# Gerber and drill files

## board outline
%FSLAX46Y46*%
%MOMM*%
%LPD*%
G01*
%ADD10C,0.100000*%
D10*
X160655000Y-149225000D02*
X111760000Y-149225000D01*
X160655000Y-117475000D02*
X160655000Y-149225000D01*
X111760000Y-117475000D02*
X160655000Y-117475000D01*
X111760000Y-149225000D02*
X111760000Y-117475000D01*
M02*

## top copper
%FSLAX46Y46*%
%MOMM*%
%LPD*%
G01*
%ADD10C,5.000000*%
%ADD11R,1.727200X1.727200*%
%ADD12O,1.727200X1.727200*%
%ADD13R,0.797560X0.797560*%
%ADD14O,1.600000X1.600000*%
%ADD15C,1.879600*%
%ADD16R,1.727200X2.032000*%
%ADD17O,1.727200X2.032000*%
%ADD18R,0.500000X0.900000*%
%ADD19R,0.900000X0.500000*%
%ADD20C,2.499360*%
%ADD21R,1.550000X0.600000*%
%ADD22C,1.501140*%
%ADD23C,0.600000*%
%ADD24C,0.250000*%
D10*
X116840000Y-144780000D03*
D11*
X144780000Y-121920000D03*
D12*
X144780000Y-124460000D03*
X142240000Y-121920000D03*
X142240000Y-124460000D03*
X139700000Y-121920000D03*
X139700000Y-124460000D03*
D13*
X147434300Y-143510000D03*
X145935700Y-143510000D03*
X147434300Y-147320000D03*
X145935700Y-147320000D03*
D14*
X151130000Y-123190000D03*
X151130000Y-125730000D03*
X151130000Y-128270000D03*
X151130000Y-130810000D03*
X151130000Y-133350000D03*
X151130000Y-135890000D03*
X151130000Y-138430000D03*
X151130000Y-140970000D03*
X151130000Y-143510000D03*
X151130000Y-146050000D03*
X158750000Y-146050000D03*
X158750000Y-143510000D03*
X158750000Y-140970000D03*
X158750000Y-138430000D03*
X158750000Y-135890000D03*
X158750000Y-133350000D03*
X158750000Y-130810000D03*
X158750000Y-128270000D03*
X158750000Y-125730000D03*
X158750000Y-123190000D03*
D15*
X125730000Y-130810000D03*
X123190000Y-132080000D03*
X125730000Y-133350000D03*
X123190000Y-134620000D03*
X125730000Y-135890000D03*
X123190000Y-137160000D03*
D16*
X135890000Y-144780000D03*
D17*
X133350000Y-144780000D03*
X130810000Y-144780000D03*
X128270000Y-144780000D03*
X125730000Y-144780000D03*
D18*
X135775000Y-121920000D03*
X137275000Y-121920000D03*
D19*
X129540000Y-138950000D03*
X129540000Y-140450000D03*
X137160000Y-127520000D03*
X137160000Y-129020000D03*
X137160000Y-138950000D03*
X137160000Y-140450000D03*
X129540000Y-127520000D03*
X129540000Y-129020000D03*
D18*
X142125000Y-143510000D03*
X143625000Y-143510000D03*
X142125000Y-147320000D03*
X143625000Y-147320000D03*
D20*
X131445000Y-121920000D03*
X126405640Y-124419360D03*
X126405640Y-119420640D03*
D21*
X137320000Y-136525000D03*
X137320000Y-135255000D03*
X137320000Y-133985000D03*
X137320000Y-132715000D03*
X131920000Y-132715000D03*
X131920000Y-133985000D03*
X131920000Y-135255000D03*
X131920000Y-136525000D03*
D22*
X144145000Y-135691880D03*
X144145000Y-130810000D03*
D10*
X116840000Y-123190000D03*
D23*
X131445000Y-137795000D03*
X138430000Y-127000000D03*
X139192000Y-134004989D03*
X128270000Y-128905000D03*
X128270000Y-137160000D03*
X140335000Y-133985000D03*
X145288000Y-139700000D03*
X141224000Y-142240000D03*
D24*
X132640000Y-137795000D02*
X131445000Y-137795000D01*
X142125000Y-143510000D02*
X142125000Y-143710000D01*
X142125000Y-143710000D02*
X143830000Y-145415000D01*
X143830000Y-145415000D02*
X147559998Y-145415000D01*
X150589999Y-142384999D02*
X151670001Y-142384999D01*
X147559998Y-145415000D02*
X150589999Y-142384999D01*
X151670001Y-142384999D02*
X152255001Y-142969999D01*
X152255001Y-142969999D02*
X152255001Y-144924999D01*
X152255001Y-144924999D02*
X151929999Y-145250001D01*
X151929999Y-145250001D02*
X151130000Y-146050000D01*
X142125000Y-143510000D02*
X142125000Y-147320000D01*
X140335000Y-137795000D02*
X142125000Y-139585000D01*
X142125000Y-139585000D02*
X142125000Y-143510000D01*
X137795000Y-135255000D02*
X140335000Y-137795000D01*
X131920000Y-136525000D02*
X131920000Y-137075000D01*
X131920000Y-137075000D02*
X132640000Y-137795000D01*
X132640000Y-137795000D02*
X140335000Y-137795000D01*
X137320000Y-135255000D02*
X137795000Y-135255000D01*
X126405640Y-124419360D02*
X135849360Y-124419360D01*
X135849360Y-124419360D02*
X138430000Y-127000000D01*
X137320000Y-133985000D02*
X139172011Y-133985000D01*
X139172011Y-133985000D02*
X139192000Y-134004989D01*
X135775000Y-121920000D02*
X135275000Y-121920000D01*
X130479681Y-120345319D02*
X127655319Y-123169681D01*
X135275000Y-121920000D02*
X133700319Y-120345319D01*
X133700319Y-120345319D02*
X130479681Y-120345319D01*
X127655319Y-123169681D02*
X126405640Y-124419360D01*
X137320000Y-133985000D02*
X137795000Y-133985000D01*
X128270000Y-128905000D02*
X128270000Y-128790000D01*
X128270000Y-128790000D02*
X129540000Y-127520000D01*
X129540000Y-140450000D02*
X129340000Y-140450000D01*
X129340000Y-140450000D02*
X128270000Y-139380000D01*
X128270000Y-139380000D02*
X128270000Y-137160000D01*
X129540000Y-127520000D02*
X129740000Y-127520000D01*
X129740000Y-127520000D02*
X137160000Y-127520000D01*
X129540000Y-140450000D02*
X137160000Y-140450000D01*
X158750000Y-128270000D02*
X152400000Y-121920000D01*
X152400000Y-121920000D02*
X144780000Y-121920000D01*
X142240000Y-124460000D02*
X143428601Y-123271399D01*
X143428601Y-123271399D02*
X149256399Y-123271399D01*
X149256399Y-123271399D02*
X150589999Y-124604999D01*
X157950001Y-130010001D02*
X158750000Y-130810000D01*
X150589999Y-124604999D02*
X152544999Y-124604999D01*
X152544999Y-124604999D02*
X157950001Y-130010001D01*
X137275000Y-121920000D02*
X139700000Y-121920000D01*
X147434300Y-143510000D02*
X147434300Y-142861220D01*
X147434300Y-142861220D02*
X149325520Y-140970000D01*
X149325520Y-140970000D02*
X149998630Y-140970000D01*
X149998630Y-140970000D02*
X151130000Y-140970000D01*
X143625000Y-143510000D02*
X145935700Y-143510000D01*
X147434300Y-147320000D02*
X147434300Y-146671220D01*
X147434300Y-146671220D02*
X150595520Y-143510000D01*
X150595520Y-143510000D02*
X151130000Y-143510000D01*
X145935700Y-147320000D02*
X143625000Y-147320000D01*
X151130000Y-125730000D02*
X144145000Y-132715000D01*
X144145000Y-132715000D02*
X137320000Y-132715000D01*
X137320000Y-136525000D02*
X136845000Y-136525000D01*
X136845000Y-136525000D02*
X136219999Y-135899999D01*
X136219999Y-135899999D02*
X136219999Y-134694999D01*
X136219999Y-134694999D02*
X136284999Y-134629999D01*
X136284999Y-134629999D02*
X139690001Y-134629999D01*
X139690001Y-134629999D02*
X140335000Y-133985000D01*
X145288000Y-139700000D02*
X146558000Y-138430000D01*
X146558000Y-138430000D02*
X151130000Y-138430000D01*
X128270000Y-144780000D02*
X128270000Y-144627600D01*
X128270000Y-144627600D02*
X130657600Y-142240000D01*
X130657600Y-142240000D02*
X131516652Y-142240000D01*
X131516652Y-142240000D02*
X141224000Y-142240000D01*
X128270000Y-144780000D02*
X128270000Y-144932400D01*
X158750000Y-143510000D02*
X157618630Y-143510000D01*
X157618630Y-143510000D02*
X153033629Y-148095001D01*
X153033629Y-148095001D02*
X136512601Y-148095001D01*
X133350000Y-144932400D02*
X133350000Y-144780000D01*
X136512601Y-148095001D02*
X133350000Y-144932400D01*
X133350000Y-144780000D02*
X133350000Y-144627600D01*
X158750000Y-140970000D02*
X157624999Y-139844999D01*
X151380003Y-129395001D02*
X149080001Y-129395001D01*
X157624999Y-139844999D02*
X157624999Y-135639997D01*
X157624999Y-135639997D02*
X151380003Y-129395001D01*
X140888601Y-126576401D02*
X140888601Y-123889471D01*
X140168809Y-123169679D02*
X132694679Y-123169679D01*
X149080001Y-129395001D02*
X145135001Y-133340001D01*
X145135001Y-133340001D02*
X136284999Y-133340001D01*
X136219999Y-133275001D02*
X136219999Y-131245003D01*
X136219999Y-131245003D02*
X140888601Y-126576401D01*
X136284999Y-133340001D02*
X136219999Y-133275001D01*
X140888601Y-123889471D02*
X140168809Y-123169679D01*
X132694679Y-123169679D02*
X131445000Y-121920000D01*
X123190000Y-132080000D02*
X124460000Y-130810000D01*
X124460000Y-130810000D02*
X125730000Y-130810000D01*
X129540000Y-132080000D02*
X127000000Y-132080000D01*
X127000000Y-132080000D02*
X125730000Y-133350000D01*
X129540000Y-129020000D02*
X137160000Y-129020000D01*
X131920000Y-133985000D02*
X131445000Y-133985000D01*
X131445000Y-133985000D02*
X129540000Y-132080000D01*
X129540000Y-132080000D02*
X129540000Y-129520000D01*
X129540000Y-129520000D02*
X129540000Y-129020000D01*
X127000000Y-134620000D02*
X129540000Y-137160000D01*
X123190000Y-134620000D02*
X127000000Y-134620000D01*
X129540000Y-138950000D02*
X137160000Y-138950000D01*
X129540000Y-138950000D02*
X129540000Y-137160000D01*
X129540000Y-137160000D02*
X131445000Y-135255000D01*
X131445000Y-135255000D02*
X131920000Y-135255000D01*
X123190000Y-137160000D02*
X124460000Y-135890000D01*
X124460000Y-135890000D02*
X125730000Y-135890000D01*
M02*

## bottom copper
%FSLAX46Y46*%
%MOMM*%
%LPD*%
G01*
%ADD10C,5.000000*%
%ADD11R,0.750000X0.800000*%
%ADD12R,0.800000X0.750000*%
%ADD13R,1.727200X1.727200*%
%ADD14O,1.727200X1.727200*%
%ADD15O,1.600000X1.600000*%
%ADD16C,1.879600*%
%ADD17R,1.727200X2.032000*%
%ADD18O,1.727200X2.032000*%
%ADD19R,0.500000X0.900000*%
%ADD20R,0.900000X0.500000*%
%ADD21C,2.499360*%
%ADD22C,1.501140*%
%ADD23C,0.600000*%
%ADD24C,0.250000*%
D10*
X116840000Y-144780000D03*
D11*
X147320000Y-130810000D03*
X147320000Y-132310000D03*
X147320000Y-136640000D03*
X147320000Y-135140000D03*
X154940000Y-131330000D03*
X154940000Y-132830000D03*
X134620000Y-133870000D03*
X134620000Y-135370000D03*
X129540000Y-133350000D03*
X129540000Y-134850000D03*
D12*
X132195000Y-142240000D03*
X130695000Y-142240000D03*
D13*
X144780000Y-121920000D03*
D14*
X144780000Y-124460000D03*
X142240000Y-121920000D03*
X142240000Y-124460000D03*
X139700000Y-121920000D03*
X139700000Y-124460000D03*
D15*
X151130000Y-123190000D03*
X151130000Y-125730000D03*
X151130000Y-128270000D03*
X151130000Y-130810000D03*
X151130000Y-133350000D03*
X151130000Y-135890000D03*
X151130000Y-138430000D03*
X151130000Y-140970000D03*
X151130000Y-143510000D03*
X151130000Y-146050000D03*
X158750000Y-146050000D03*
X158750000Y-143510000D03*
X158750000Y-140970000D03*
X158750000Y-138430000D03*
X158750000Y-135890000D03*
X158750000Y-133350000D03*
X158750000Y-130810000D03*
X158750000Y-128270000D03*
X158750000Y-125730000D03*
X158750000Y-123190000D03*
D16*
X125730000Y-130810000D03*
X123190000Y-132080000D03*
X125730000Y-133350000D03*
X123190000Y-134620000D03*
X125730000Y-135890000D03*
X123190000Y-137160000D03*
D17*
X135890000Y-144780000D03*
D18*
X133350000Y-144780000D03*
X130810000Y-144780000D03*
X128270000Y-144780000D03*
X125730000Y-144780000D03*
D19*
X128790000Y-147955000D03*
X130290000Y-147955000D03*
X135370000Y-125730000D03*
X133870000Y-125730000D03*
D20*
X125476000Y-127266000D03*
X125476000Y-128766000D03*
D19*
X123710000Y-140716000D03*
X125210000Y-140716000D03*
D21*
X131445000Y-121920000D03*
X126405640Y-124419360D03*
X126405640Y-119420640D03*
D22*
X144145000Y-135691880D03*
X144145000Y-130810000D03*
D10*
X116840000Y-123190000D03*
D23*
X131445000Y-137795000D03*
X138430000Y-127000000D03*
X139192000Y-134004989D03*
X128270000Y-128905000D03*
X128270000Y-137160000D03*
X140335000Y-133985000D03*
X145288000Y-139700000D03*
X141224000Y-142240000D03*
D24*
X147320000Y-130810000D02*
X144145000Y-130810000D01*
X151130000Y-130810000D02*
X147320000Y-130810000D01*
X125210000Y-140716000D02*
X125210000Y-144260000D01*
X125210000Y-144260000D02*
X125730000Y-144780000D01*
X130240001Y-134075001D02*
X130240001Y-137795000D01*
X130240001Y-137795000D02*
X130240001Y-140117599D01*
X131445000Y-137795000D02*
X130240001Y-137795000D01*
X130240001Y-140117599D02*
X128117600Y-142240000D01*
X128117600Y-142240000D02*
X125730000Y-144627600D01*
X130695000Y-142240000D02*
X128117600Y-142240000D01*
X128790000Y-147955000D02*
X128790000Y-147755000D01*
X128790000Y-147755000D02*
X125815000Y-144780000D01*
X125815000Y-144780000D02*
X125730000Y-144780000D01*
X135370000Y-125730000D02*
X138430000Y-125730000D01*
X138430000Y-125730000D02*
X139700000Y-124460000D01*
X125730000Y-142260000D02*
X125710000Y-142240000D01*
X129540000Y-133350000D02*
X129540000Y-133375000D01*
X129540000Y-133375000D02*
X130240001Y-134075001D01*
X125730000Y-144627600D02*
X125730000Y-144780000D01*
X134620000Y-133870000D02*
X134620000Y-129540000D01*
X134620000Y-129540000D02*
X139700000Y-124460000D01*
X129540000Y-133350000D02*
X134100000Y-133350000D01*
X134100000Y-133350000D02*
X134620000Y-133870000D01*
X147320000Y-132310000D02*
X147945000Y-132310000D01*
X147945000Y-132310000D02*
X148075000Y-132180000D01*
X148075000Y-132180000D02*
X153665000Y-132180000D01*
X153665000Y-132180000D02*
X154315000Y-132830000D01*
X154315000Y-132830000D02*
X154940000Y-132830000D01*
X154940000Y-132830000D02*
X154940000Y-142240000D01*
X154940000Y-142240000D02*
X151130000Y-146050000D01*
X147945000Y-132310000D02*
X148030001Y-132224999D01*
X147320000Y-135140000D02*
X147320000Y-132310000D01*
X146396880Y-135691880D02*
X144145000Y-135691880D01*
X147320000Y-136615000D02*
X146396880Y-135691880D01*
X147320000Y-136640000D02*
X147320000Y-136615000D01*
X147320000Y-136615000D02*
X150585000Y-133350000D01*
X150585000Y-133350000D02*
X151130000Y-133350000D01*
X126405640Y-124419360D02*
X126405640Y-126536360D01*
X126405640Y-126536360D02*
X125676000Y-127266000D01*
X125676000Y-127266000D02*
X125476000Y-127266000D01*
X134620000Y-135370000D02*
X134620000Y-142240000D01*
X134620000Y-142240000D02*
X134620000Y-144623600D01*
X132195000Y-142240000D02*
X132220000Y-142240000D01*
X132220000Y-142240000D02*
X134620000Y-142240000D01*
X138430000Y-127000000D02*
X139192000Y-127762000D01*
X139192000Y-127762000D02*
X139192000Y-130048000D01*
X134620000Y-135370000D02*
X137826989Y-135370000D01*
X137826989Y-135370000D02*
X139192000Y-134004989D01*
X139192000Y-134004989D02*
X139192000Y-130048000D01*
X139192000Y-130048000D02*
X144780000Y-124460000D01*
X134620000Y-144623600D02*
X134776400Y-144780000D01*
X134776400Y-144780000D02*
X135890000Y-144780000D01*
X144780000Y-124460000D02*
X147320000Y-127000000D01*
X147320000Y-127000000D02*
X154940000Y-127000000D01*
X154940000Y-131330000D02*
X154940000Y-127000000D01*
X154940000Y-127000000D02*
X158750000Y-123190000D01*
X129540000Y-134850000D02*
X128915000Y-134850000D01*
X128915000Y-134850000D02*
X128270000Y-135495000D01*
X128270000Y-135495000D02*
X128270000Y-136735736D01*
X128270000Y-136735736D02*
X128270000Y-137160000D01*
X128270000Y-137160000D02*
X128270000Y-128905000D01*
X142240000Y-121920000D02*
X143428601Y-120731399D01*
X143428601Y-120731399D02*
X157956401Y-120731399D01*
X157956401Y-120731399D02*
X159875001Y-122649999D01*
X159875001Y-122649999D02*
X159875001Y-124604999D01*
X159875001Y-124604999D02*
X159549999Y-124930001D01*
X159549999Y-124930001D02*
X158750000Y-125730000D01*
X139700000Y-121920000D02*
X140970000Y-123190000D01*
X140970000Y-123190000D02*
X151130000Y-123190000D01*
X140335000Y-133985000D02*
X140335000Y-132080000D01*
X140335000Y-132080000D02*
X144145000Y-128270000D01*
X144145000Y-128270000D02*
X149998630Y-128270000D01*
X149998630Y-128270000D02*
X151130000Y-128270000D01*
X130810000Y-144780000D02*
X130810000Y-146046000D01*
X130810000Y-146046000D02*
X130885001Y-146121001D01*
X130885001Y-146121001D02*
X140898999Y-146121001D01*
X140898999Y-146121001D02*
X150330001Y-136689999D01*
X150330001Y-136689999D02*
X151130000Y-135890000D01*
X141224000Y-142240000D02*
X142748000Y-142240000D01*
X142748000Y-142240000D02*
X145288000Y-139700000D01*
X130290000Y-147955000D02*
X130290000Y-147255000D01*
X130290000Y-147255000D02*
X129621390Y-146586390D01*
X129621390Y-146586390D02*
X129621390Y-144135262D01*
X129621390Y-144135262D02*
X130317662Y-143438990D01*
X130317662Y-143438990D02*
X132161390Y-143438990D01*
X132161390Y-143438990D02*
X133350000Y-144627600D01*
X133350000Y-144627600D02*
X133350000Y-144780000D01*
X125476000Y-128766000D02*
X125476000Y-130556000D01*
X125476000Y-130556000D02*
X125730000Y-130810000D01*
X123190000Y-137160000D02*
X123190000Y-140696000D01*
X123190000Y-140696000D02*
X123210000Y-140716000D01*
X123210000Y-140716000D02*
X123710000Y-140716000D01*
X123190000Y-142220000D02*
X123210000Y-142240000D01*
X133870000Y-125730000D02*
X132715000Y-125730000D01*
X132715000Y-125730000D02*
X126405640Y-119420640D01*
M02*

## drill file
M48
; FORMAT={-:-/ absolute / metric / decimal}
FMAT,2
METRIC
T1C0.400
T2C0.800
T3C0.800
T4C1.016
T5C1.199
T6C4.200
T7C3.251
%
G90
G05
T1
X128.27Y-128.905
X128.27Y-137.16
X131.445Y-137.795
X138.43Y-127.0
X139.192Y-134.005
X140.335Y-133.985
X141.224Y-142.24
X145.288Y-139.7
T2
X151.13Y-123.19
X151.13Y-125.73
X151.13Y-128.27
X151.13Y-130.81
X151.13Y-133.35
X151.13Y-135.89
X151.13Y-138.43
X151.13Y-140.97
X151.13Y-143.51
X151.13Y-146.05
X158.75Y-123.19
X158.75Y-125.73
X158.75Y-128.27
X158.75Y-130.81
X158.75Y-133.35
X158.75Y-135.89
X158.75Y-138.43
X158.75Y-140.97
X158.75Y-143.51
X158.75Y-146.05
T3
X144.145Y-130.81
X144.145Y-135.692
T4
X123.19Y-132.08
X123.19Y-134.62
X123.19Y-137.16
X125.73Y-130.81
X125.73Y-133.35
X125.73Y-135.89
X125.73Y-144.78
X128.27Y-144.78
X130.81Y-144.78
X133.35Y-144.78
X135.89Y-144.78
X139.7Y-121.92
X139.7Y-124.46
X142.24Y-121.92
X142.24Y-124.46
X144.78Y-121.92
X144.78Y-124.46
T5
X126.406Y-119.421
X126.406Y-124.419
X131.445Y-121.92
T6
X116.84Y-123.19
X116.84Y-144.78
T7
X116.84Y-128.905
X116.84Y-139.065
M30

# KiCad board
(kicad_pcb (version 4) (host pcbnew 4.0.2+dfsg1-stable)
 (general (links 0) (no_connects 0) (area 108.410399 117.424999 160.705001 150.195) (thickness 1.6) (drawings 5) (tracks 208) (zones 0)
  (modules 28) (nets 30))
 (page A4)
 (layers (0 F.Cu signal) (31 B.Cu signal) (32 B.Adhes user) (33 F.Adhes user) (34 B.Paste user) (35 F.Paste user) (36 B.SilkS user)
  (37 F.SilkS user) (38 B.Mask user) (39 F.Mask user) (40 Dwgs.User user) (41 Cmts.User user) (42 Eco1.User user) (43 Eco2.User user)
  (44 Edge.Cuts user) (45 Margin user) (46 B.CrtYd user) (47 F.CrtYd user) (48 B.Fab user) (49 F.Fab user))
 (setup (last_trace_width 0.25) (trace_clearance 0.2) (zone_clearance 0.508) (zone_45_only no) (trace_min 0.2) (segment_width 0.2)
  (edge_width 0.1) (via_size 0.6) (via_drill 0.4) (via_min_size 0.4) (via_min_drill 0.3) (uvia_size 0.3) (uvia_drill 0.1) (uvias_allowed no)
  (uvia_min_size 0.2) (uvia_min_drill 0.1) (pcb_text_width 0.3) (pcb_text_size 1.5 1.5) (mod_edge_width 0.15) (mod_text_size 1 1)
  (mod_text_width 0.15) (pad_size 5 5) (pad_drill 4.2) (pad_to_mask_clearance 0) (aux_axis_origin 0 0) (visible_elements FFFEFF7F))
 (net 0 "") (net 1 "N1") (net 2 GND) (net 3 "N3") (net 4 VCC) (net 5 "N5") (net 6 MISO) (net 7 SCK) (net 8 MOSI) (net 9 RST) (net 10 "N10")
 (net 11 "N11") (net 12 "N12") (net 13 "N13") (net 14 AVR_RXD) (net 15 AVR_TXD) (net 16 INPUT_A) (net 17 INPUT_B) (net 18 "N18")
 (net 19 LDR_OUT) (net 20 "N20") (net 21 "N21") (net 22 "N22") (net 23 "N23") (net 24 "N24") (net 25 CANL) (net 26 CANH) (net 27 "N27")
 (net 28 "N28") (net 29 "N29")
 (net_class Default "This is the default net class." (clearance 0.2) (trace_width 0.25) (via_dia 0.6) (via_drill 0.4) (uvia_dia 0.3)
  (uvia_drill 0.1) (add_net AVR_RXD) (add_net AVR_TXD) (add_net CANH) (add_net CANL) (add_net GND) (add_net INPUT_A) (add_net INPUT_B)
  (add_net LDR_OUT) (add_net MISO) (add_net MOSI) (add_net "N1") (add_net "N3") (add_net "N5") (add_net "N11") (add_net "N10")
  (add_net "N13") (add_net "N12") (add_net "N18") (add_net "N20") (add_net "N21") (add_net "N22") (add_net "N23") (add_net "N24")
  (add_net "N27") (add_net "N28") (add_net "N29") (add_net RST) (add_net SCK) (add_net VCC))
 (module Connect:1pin (layer F.Cu) (at 116.84 144.78)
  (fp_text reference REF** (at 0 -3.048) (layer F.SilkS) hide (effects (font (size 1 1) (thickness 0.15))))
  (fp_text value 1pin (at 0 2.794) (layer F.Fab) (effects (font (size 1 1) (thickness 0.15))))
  (pad 1 thru_hole circle (at 0 0) (size 5 5) (drill 4.2) (layers *.Cu *.Mask F.SilkS)))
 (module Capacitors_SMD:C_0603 (layer B.Cu) (at 147.32 131.56 270)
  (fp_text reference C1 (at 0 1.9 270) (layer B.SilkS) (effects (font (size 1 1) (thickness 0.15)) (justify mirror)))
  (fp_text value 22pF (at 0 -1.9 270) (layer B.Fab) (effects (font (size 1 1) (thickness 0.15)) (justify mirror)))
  (pad 1 smd rect (at -0.75 0 270) (size 0.8 0.75) (layers B.Cu B.Paste B.Mask) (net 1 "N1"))
  (pad 2 smd rect (at 0.75 0 270) (size 0.8 0.75) (layers B.Cu B.Paste B.Mask) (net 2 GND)))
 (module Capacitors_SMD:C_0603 (layer B.Cu) (at 147.32 135.89 90)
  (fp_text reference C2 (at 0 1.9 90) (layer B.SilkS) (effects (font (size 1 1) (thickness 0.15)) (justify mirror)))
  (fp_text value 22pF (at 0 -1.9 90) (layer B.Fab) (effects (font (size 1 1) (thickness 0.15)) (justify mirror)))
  (pad 1 smd rect (at -0.75 0 90) (size 0.8 0.75) (layers B.Cu B.Paste B.Mask) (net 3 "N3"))
  (pad 2 smd rect (at 0.75 0 90) (size 0.8 0.75) (layers B.Cu B.Paste B.Mask) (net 2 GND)))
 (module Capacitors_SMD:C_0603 (layer B.Cu) (at 154.94 132.08 270)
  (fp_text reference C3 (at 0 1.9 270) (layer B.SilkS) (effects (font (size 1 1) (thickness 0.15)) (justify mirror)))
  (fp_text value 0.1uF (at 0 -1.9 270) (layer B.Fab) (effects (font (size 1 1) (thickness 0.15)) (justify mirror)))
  (pad 1 smd rect (at -0.75 0 270) (size 0.8 0.75) (layers B.Cu B.Paste B.Mask) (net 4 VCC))
  (pad 2 smd rect (at 0.75 0 270) (size 0.8 0.75) (layers B.Cu B.Paste B.Mask) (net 2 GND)))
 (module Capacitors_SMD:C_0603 (layer B.Cu) (at 134.62 134.62 270)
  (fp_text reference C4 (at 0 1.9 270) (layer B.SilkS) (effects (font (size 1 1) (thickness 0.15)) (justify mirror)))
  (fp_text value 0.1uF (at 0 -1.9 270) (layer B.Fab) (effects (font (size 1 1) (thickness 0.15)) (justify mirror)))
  (pad 1 smd rect (at -0.75 0 270) (size 0.8 0.75) (layers B.Cu B.Paste B.Mask) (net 2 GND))
  (pad 2 smd rect (at 0.75 0 270) (size 0.8 0.75) (layers B.Cu B.Paste B.Mask) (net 4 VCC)))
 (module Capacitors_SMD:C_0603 (layer B.Cu) (at 129.54 134.1 270)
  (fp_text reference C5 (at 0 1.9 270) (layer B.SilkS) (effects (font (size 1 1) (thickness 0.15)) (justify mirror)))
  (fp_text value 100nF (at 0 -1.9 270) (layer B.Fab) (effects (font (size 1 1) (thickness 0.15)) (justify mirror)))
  (pad 1 smd rect (at -0.75 0 270) (size 0.8 0.75) (layers B.Cu B.Paste B.Mask) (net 2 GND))
  (pad 2 smd rect (at 0.75 0 270) (size 0.8 0.75) (layers B.Cu B.Paste B.Mask) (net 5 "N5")))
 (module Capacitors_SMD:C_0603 (layer B.Cu) (at 131.445 142.24 180)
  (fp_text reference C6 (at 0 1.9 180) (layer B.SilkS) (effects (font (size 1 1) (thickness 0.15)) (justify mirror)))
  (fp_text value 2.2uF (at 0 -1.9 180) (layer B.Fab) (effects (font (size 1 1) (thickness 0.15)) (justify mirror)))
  (pad 1 smd rect (at -0.75 0 180) (size 0.8 0.75) (layers B.Cu B.Paste B.Mask) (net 4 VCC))
  (pad 2 smd rect (at 0.75 0 180) (size 0.8 0.75) (layers B.Cu B.Paste B.Mask) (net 2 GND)))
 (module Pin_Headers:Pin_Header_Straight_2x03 (layer F.Cu) (at 144.78 121.92 270)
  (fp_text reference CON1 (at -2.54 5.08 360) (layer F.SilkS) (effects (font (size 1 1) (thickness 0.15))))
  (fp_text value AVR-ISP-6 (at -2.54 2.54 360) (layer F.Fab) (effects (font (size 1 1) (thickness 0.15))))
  (pad 1 thru_hole rect (at 0 0 270) (size 1.7272 1.7272) (drill 1.016) (layers *.Cu *.Mask F.SilkS) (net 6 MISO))
  (pad 2 thru_hole oval (at 2.54 0 270) (size 1.7272 1.7272) (drill 1.016) (layers *.Cu *.Mask F.SilkS) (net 4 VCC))
  (pad 3 thru_hole oval (at 0 2.54 270) (size 1.7272 1.7272) (drill 1.016) (layers *.Cu *.Mask F.SilkS) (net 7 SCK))
  (pad 4 thru_hole oval (at 2.54 2.54 270) (size 1.7272 1.7272) (drill 1.016) (layers *.Cu *.Mask F.SilkS) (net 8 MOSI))
  (pad 5 thru_hole oval (at 0 5.08 270) (size 1.7272 1.7272) (drill 1.016) (layers *.Cu *.Mask F.SilkS) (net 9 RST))
  (pad 6 thru_hole oval (at 2.54 5.08 270) (size 1.7272 1.7272) (drill 1.016) (layers *.Cu *.Mask F.SilkS) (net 2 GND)))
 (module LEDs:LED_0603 (layer F.Cu) (at 146.685 143.51)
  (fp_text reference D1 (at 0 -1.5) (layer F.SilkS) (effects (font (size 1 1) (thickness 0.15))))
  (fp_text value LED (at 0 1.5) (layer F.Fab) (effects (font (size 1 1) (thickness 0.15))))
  (pad 2 smd rect (at 0.7493 0 180) (size 0.79756 0.79756) (layers F.Cu F.Paste F.Mask) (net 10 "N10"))
  (pad 1 smd rect (at -0.7493 0 180) (size 0.79756 0.79756) (layers F.Cu F.Paste F.Mask) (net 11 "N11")))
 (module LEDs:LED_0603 (layer F.Cu) (at 146.685 147.32)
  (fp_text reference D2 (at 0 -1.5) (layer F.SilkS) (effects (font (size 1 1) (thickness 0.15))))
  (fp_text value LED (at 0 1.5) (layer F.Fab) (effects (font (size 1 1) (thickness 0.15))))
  (pad 2 smd rect (at 0.7493 0 180) (size 0.79756 0.79756) (layers F.Cu F.Paste F.Mask) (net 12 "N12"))
  (pad 1 smd rect (at -0.7493 0 180) (size 0.79756 0.79756) (layers F.Cu F.Paste F.Mask) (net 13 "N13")))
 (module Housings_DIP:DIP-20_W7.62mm (layer F.Cu) (at 151.13 123.19)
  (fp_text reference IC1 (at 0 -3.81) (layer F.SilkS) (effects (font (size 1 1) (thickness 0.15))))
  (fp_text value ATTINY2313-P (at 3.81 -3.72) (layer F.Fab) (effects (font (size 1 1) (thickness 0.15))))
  (pad 1 thru_hole oval (at 0 0) (size 1.6 1.6) (drill 0.8) (layers *.Cu *.Mask F.SilkS) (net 9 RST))
  (pad 2 thru_hole oval (at 0 2.54) (size 1.6 1.6) (drill 0.8) (layers *.Cu *.Mask F.SilkS) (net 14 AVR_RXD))
  (pad 3 thru_hole oval (at 0 5.08) (size 1.6 1.6) (drill 0.8) (layers *.Cu *.Mask F.SilkS) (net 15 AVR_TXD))
  (pad 4 thru_hole oval (at 0 7.62) (size 1.6 1.6) (drill 0.8) (layers *.Cu *.Mask F.SilkS) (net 1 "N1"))
  (pad 5 thru_hole oval (at 0 10.16) (size 1.6 1.6) (drill 0.8) (layers *.Cu *.Mask F.SilkS) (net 3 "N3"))
  (pad 6 thru_hole oval (at 0 12.7) (size 1.6 1.6) (drill 0.8) (layers *.Cu *.Mask F.SilkS) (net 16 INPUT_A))
  (pad 7 thru_hole oval (at 0 15.24) (size 1.6 1.6) (drill 0.8) (layers *.Cu *.Mask F.SilkS) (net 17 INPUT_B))
  (pad 8 thru_hole oval (at 0 17.78) (size 1.6 1.6) (drill 0.8) (layers *.Cu *.Mask F.SilkS) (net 10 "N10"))
  (pad 9 thru_hole oval (at 0 20.32) (size 1.6 1.6) (drill 0.8) (layers *.Cu *.Mask F.SilkS) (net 12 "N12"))
  (pad 10 thru_hole oval (at 0 22.86) (size 1.6 1.6) (drill 0.8) (layers *.Cu *.Mask F.SilkS) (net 2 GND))
  (pad 11 thru_hole oval (at 7.62 22.86) (size 1.6 1.6) (drill 0.8) (layers *.Cu *.Mask F.SilkS) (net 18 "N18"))
  (pad 12 thru_hole oval (at 7.62 20.32) (size 1.6 1.6) (drill 0.8) (layers *.Cu *.Mask F.SilkS) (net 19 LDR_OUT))
  (pad 13 thru_hole oval (at 7.62 17.78) (size 1.6 1.6) (drill 0.8) (layers *.Cu *.Mask F.SilkS) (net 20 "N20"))
  (pad 14 thru_hole oval (at 7.62 15.24) (size 1.6 1.6) (drill 0.8) (layers *.Cu *.Mask F.SilkS) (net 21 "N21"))
  (pad 15 thru_hole oval (at 7.62 12.7) (size 1.6 1.6) (drill 0.8) (layers *.Cu *.Mask F.SilkS) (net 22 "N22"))
  (pad 16 thru_hole oval (at 7.62 10.16) (size 1.6 1.6) (drill 0.8) (layers *.Cu *.Mask F.SilkS) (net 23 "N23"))
  (pad 17 thru_hole oval (at 7.62 7.62) (size 1.6 1.6) (drill 0.8) (layers *.Cu *.Mask F.SilkS) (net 8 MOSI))
  (pad 18 thru_hole oval (at 7.62 5.08) (size 1.6 1.6) (drill 0.8) (layers *.Cu *.Mask F.SilkS) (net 6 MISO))
  (pad 19 thru_hole oval (at 7.62 2.54) (size 1.6 1.6) (drill 0.8) (layers *.Cu *.Mask F.SilkS) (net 7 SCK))
  (pad 20 thru_hole oval (at 7.62 0) (size 1.6 1.6) (drill 0.8) (layers *.Cu *.Mask F.SilkS) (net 4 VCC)))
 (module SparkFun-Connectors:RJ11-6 (layer F.Cu) (at 116.84 133.985 270)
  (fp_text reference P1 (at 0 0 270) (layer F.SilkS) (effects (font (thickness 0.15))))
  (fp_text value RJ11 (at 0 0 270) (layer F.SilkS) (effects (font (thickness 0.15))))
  (pad 1 thru_hole circle (at -3.175 -8.89 270) (size 1.8796 1.8796) (drill 1.016) (layers *.Cu *.Mask) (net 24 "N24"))
  (pad 2 thru_hole circle (at -1.905 -6.35 270) (size 1.8796 1.8796) (drill 1.016) (layers *.Cu *.Mask) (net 24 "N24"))
  (pad 3 thru_hole circle (at -0.635 -8.89 270) (size 1.8796 1.8796) (drill 1.016) (layers *.Cu *.Mask) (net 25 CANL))
  (pad 4 thru_hole circle (at 0.635 -6.35 270) (size 1.8796 1.8796) (drill 1.016) (layers *.Cu *.Mask) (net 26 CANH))
  (pad 5 thru_hole circle (at 1.905 -8.89 270) (size 1.8796 1.8796) (drill 1.016) (layers *.Cu *.Mask) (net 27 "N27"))
  (pad 6 thru_hole circle (at 3.175 -6.35 270) (size 1.8796 1.8796) (drill 1.016) (layers *.Cu *.Mask) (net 27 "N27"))
  (pad "" np_thru_hole circle (at -5.08 0 270) (size 3.2512 3.2512) (drill 3.2512) (layers *.Cu))
  (pad "" np_thru_hole circle (at 5.08 0 270) (size 3.2512 3.2512) (drill 3.2512) (layers *.Cu)))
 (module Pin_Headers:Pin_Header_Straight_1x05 (layer F.Cu) (at 135.89 144.78 270)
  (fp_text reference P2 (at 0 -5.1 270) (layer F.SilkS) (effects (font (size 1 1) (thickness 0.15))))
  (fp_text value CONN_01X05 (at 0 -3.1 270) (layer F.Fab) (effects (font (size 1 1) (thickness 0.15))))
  (pad 1 thru_hole rect (at 0 0 270) (size 2.032 1.7272) (drill 1.016) (layers *.Cu *.Mask F.SilkS) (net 4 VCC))
  (pad 2 thru_hole oval (at 0 2.54 270) (size 2.032 1.7272) (drill 1.016) (layers *.Cu *.Mask F.SilkS) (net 19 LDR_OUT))
  (pad 3 thru_hole oval (at 0 5.08 270) (size 2.032 1.7272) (drill 1.016) (layers *.Cu *.Mask F.SilkS) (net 16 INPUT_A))
  (pad 4 thru_hole oval (at 0 7.62 270) (size 2.032 1.7272) (drill 1.016) (layers *.Cu *.Mask F.SilkS) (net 17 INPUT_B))
  (pad 5 thru_hole oval (at 0 10.16 270) (size 2.032 1.7272) (drill 1.016) (layers *.Cu *.Mask F.SilkS) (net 2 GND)))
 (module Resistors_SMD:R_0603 (layer F.Cu) (at 136.525 121.92)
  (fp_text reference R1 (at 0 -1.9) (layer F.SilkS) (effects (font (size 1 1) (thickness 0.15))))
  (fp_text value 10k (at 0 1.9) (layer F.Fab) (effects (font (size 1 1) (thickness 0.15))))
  (pad 1 smd rect (at -0.75 0) (size 0.5 0.9) (layers F.Cu F.Paste F.Mask) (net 4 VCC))
  (pad 2 smd rect (at 0.75 0) (size 0.5 0.9) (layers F.Cu F.Paste F.Mask) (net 9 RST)))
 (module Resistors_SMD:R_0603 (layer B.Cu) (at 129.54 147.955)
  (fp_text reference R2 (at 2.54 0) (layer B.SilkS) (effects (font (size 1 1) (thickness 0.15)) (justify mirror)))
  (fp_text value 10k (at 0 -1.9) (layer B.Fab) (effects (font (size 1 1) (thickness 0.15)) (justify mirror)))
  (pad 1 smd rect (at -0.75 0) (size 0.5 0.9) (layers B.Cu B.Paste B.Mask) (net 2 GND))
  (pad 2 smd rect (at 0.75 0) (size 0.5 0.9) (layers B.Cu B.Paste B.Mask) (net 19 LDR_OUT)))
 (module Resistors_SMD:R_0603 (layer F.Cu) (at 129.54 139.7 270)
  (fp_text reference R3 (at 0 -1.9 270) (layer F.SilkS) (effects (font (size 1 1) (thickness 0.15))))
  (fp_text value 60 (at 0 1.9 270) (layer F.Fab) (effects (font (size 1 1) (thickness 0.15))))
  (pad 1 smd rect (at -0.75 0 270) (size 0.5 0.9) (layers F.Cu F.Paste F.Mask) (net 26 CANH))
  (pad 2 smd rect (at 0.75 0 270) (size 0.5 0.9) (layers F.Cu F.Paste F.Mask) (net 5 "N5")))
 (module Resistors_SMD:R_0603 (layer F.Cu) (at 137.16 128.27 270)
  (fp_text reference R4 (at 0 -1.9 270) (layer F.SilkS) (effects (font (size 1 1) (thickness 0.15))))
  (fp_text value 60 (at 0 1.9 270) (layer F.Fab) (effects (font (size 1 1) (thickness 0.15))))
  (pad 1 smd rect (at -0.75 0 270) (size 0.5 0.9) (layers F.Cu F.Paste F.Mask) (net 5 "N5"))
  (pad 2 smd rect (at 0.75 0 270) (size 0.5 0.9) (layers F.Cu F.Paste F.Mask) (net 25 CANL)))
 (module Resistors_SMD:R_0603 (layer F.Cu) (at 137.16 139.7 270)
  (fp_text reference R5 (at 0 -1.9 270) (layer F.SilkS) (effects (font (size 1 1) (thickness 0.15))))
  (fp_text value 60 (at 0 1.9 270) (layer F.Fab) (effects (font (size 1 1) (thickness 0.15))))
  (pad 1 smd rect (at -0.75 0 270) (size 0.5 0.9) (layers F.Cu F.Paste F.Mask) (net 26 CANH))
  (pad 2 smd rect (at 0.75 0 270) (size 0.5 0.9) (layers F.Cu F.Paste F.Mask) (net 5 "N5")))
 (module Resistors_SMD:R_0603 (layer F.Cu) (at 129.54 128.27 270)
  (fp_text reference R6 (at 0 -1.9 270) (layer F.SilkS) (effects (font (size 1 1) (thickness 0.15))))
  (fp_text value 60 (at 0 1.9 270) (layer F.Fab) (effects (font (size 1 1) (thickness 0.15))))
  (pad 1 smd rect (at -0.75 0 270) (size 0.5 0.9) (layers F.Cu F.Paste F.Mask) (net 5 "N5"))
  (pad 2 smd rect (at 0.75 0 270) (size 0.5 0.9) (layers F.Cu F.Paste F.Mask) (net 25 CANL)))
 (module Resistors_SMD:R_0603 (layer B.Cu) (at 134.62 125.73 180)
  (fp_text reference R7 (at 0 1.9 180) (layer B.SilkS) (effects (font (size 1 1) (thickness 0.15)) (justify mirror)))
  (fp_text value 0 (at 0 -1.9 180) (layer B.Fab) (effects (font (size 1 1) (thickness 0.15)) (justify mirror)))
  (pad 1 smd rect (at -0.75 0 180) (size 0.5 0.9) (layers B.Cu B.Paste B.Mask) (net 2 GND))
  (pad 2 smd rect (at 0.75 0 180) (size 0.5 0.9) (layers B.Cu B.Paste B.Mask) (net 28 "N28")))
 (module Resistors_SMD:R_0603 (layer F.Cu) (at 142.875 143.51)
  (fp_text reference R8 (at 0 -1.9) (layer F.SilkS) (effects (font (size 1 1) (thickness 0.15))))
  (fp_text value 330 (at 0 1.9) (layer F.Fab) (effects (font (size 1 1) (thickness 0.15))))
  (pad 1 smd rect (at -0.75 0) (size 0.5 0.9) (layers F.Cu F.Paste F.Mask) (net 2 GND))
  (pad 2 smd rect (at 0.75 0) (size 0.5 0.9) (layers F.Cu F.Paste F.Mask) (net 11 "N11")))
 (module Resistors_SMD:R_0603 (layer F.Cu) (at 142.875 147.32)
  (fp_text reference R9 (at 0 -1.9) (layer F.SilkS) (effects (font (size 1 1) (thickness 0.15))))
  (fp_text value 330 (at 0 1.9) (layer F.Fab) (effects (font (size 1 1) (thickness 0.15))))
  (pad 1 smd rect (at -0.75 0) (size 0.5 0.9) (layers F.Cu F.Paste F.Mask) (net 2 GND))
  (pad 2 smd rect (at 0.75 0) (size 0.5 0.9) (layers F.Cu F.Paste F.Mask) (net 13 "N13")))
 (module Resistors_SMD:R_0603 (layer B.Cu) (at 125.476 128.016 270)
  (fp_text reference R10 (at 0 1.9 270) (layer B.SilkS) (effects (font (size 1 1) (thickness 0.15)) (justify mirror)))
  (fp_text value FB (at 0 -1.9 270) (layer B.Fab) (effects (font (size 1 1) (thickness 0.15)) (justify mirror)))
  (pad 1 smd rect (at -0.75 0 270) (size 0.5 0.9) (layers B.Cu B.Paste B.Mask) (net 4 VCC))
  (pad 2 smd rect (at 0.75 0 270) (size 0.5 0.9) (layers B.Cu B.Paste B.Mask) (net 24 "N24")))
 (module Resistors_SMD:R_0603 (layer B.Cu) (at 124.46 140.716)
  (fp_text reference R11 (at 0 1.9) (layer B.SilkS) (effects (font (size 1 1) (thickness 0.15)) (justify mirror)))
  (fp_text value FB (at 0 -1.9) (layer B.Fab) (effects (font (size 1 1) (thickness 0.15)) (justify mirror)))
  (pad 1 smd rect (at -0.75 0) (size 0.5 0.9) (layers B.Cu B.Paste B.Mask) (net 27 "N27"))
  (pad 2 smd rect (at 0.75 0) (size 0.5 0.9) (layers B.Cu B.Paste B.Mask) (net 2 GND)))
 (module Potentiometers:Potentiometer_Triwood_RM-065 (layer F.Cu) (at 126.40564 119.42064 270)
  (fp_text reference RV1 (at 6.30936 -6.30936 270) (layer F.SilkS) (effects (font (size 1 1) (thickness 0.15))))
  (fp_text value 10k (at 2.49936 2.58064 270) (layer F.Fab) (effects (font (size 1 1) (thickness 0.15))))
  (pad 2 thru_hole circle (at 2.49936 -5.03936 270) (size 2.49936 2.49936) (drill 1.19888) (layers *.Cu *.Mask F.SilkS) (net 20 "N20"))
  (pad 3 thru_hole circle (at 4.99872 0 270) (size 2.49936 2.49936) (drill 1.19888) (layers *.Cu *.Mask F.SilkS) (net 4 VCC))
  (pad 1 thru_hole circle (at 0 0 270) (size 2.49936 2.49936) (drill 1.19888) (layers *.Cu *.Mask F.SilkS) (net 28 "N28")))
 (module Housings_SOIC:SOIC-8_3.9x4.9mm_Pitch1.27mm (layer F.Cu) (at 134.62 134.62 180)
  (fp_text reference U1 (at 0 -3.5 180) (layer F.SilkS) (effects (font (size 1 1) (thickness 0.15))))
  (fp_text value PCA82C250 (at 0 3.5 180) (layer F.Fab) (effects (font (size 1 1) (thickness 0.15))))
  (pad 1 smd rect (at -2.7 -1.905 180) (size 1.55 0.6) (layers F.Cu F.Paste F.Mask) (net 15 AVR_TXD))
  (pad 2 smd rect (at -2.7 -0.635 180) (size 1.55 0.6) (layers F.Cu F.Paste F.Mask) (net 2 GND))
  (pad 3 smd rect (at -2.7 0.635 180) (size 1.55 0.6) (layers F.Cu F.Paste F.Mask) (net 4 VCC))
  (pad 4 smd rect (at -2.7 1.905 180) (size 1.55 0.6) (layers F.Cu F.Paste F.Mask) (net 14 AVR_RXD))
  (pad 5 smd rect (at 2.7 1.905 180) (size 1.55 0.6) (layers F.Cu F.Paste F.Mask) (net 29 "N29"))
  (pad 6 smd rect (at 2.7 0.635 180) (size 1.55 0.6) (layers F.Cu F.Paste F.Mask) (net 25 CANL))
  (pad 7 smd rect (at 2.7 -0.635 180) (size 1.55 0.6) (layers F.Cu F.Paste F.Mask) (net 26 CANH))
  (pad 8 smd rect (at 2.7 -1.905 180) (size 1.55 0.6) (layers F.Cu F.Paste F.Mask) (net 2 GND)))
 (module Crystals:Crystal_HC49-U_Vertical (layer F.Cu) (at 144.145 133.25094 90)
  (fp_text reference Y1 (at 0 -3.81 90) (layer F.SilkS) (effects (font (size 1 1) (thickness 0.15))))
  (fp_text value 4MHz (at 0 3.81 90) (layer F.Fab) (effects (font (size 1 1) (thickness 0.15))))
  (pad 1 thru_hole circle (at -2.44094 0 90) (size 1.50114 1.50114) (drill 0.8001) (layers *.Cu *.Mask F.SilkS) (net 3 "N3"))
  (pad 2 thru_hole circle (at 2.44094 0 90) (size 1.50114 1.50114) (drill 0.8001) (layers *.Cu *.Mask F.SilkS) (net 1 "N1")))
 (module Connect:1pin (layer F.Cu) (at 116.84 123.19)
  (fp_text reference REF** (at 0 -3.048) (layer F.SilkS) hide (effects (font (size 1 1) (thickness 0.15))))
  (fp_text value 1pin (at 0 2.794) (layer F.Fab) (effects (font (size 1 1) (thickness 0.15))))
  (pad 1 thru_hole circle (at 0 0) (size 5 5) (drill 4.2) (layers *.Cu *.Mask F.SilkS)))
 (gr_line (start 160.655 149.225) (end 111.76 149.225) (layer Edge.Cuts) (width 0.1))
 (gr_line (start 160.655 117.475) (end 160.655 149.225) (layer Edge.Cuts) (width 0.1))
 (gr_line (start 111.76 117.475) (end 160.655 117.475) (layer Edge.Cuts) (width 0.1))
 (gr_line (start 111.76 149.225) (end 111.76 117.475) (layer Edge.Cuts) (width 0.1))
 (segment (start 147.32 130.81) (end 144.145 130.81) (width 0.25) (layer B.Cu) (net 1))
 (segment (start 151.13 130.81) (end 147.32 130.81) (width 0.25) (layer B.Cu) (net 1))
 (segment (start 125.21 140.716) (end 125.21 144.26) (width 0.25) (layer B.Cu) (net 2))
 (segment (start 125.21 144.26) (end 125.73 144.78) (width 0.25) (layer B.Cu) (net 2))
 (segment (start 130.240001 134.075001) (end 130.240001 137.795) (width 0.25) (layer B.Cu) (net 2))
 (segment (start 130.240001 137.795) (end 130.240001 140.117599) (width 0.25) (layer B.Cu) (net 2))
 (segment (start 131.445 137.795) (end 130.240001 137.795) (width 0.25) (layer B.Cu) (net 2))
 (segment (start 132.64 137.795) (end 131.445 137.795) (width 0.25) (layer F.Cu) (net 2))
 (via (at 131.445 137.795) (size 0.6) (drill 0.4) (layers F.Cu B.Cu) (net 2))
 (segment (start 130.240001 140.117599) (end 128.1176 142.24) (width 0.25) (layer B.Cu) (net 2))
 (segment (start 128.1176 142.24) (end 125.73 144.6276) (width 0.25) (layer B.Cu) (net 2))
 (segment (start 130.695 142.24) (end 128.1176 142.24) (width 0.25) (layer B.Cu) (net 2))
 (segment (start 128.79 147.955) (end 128.79 147.755) (width 0.25) (layer B.Cu) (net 2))
 (segment (start 128.79 147.755) (end 125.815 144.78) (width 0.25) (layer B.Cu) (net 2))
 (segment (start 125.815 144.78) (end 125.73 144.78) (width 0.25) (layer B.Cu) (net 2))
 (segment (start 142.125 143.51) (end 142.125 143.71) (width 0.25) (layer F.Cu) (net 2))
 (segment (start 142.125 143.71) (end 143.83 145.415) (width 0.25) (layer F.Cu) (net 2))
 (segment (start 143.83 145.415) (end 147.559998 145.415) (width 0.25) (layer F.Cu) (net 2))
 (segment (start 150.589999 142.384999) (end 151.670001 142.384999) (width 0.25) (layer F.Cu) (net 2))
 (segment (start 147.559998 145.415) (end 150.589999 142.384999) (width 0.25) (layer F.Cu) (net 2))
 (segment (start 151.670001 142.384999) (end 152.255001 142.969999) (width 0.25) (layer F.Cu) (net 2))
 (segment (start 152.255001 142.969999) (end 152.255001 144.924999) (width 0.25) (layer F.Cu) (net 2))
 (segment (start 152.255001 144.924999) (end 151.929999 145.250001) (width 0.25) (layer F.Cu) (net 2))
 (segment (start 151.929999 145.250001) (end 151.13 146.05) (width 0.25) (layer F.Cu) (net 2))
 (segment (start 135.37 125.73) (end 138.43 125.73) (width 0.25) (layer B.Cu) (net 2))
 (segment (start 138.43 125.73) (end 139.7 124.46) (width 0.25) (layer B.Cu) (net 2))
 (segment (start 125.73 142.26) (end 125.71 142.24) (width 0.25) (layer B.Cu) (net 2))
 (segment (start 129.54 133.35) (end 129.54 133.375) (width 0.25) (layer B.Cu) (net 2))
 (segment (start 129.54 133.375) (end 130.240001 134.075001) (width 0.25) (layer B.Cu) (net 2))
 (segment (start 125.73 144.6276) (end 125.73 144.78) (width 0.25) (layer B.Cu) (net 2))
 (segment (start 134.62 133.87) (end 134.62 129.54) (width 0.25) (layer B.Cu) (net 2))
 (segment (start 134.62 129.54) (end 139.7 124.46) (width 0.25) (layer B.Cu) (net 2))
 (segment (start 142.125 143.51) (end 142.125 147.32) (width 0.25) (layer F.Cu) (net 2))
 (segment (start 140.335 137.795) (end 142.125 139.585) (width 0.25) (layer F.Cu) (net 2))
 (segment (start 142.125 139.585) (end 142.125 143.51) (width 0.25) (layer F.Cu) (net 2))
 (segment (start 129.54 133.35) (end 134.1 133.35) (width 0.25) (layer B.Cu) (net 2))
 (segment (start 134.1 133.35) (end 134.62 133.87) (width 0.25) (layer B.Cu) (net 2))
 (segment (start 137.795 135.255) (end 140.335 137.795) (width 0.25) (layer F.Cu) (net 2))
 (segment (start 131.92 136.525) (end 131.92 137.075) (width 0.25) (layer F.Cu) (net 2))
 (segment (start 131.92 137.075) (end 132.64 137.795) (width 0.25) (layer F.Cu) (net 2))
 (segment (start 132.64 137.795) (end 140.335 137.795) (width 0.25) (layer F.Cu) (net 2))
 (segment (start 137.32 135.255) (end 137.795 135.255) (width 0.25) (layer F.Cu) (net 2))
 (segment (start 147.32 132.31) (end 147.945 132.31) (width 0.25) (layer B.Cu) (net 2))
 (segment (start 147.945 132.31) (end 148.075 132.18) (width 0.25) (layer B.Cu) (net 2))
 (segment (start 148.075 132.18) (end 153.665 132.18) (width 0.25) (layer B.Cu) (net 2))
 (segment (start 153.665 132.18) (end 154.315 132.83) (width 0.25) (layer B.Cu) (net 2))
 (segment (start 154.315 132.83) (end 154.94 132.83) (width 0.25) (layer B.Cu) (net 2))
 (segment (start 154.94 132.83) (end 154.94 142.24) (width 0.25) (layer B.Cu) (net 2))
 (segment (start 154.94 142.24) (end 151.13 146.05) (width 0.25) (layer B.Cu) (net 2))
 (segment (start 147.945 132.31) (end 148.030001 132.224999) (width 0.25) (layer B.Cu) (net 2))
 (segment (start 147.32 135.14) (end 147.32 132.31) (width 0.25) (layer B.Cu) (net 2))
 (segment (start 146.39688 135.69188) (end 144.145 135.69188) (width 0.25) (layer B.Cu) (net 3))
 (segment (start 147.32 136.615) (end 146.39688 135.69188) (width 0.25) (layer B.Cu) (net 3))
 (segment (start 147.32 136.64) (end 147.32 136.615) (width 0.25) (layer B.Cu) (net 3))
 (segment (start 147.32 136.615) (end 150.585 133.35) (width 0.25) (layer B.Cu) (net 3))
 (segment (start 150.585 133.35) (end 151.13 133.35) (width 0.25) (layer B.Cu) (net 3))
 (segment (start 126.40564 124.41936) (end 126.40564 126.53636) (width 0.25) (layer B.Cu) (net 4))
 (segment (start 126.40564 126.53636) (end 125.676 127.266) (width 0.25) (layer B.Cu) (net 4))
 (segment (start 125.676 127.266) (end 125.476 127.266) (width 0.25) (layer B.Cu) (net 4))
 (segment (start 134.62 135.37) (end 134.62 142.24) (width 0.25) (layer B.Cu) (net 4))
 (segment (start 134.62 142.24) (end 134.62 144.6236) (width 0.25) (layer B.Cu) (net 4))
 (segment (start 132.195 142.24) (end 132.22 142.24) (width 0.25) (layer B.Cu) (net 4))
 (segment (start 132.22 142.24) (end 134.62 142.24) (width 0.25) (layer B.Cu) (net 4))
 (segment (start 138.43 127) (end 139.192 127.762) (width 0.25) (layer B.Cu) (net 4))
 (segment (start 139.192 127.762) (end 139.192 130.048) (width 0.25) (layer B.Cu) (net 4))
 (segment (start 126.40564 124.41936) (end 135.84936 124.41936) (width 0.25) (layer F.Cu) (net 4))
 (segment (start 135.84936 124.41936) (end 138.43 127) (width 0.25) (layer F.Cu) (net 4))
 (via (at 138.43 127) (size 0.6) (drill 0.4) (layers F.Cu B.Cu) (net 4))
 (segment (start 134.62 135.37) (end 137.826989 135.37) (width 0.25) (layer B.Cu) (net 4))
 (segment (start 137.826989 135.37) (end 139.192 134.004989) (width 0.25) (layer B.Cu) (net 4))
 (segment (start 139.192 134.004989) (end 139.192 130.048) (width 0.25) (layer B.Cu) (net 4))
 (segment (start 139.192 130.048) (end 144.78 124.46) (width 0.25) (layer B.Cu) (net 4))
 (segment (start 137.32 133.985) (end 139.172011 133.985) (width 0.25) (layer F.Cu) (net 4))
 (segment (start 139.172011 133.985) (end 139.192 134.004989) (width 0.25) (layer F.Cu) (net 4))
 (via (at 139.192 134.004989) (size 0.6) (drill 0.4) (layers F.Cu B.Cu) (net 4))
 (segment (start 134.62 144.6236) (end 134.7764 144.78) (width 0.25) (layer B.Cu) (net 4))
 (segment (start 134.7764 144.78) (end 135.89 144.78) (width 0.25) (layer B.Cu) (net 4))
 (segment (start 135.775 121.92) (end 135.275 121.92) (width 0.25) (layer F.Cu) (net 4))
 (segment (start 130.479681 120.345319) (end 127.655319 123.169681) (width 0.25) (layer F.Cu) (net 4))
 (segment (start 135.275 121.92) (end 133.700319 120.345319) (width 0.25) (layer F.Cu) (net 4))
 (segment (start 133.700319 120.345319) (end 130.479681 120.345319) (width 0.25) (layer F.Cu) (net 4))
 (segment (start 127.655319 123.169681) (end 126.40564 124.41936) (width 0.25) (layer F.Cu) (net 4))
 (segment (start 144.78 124.46) (end 147.32 127) (width 0.25) (layer B.Cu) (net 4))
 (segment (start 147.32 127) (end 154.94 127) (width 0.25) (layer B.Cu) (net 4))
 (segment (start 137.32 133.985) (end 137.795 133.985) (width 0.25) (layer F.Cu) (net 4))
 (segment (start 154.94 131.33) (end 154.94 127) (width 0.25) (layer B.Cu) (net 4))
 (segment (start 154.94 127) (end 158.75 123.19) (width 0.25) (layer B.Cu) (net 4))
 (segment (start 129.54 134.85) (end 128.915 134.85) (width 0.25) (layer B.Cu) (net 5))
 (segment (start 128.915 134.85) (end 128.27 135.495) (width 0.25) (layer B.Cu) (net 5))
 (segment (start 128.27 135.495) (end 128.27 136.735736) (width 0.25) (layer B.Cu) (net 5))
 (segment (start 128.27 136.735736) (end 128.27 137.16) (width 0.25) (layer B.Cu) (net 5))
 (segment (start 128.27 128.905) (end 128.27 128.79) (width 0.25) (layer F.Cu) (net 5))
 (segment (start 128.27 128.79) (end 129.54 127.52) (width 0.25) (layer F.Cu) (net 5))
 (segment (start 128.27 137.16) (end 128.27 128.905) (width 0.25) (layer B.Cu) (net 5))
 (via (at 128.27 128.905) (size 0.6) (drill 0.4) (layers F.Cu B.Cu) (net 5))
 (segment (start 129.54 140.45) (end 129.34 140.45) (width 0.25) (layer F.Cu) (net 5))
 (segment (start 129.34 140.45) (end 128.27 139.38) (width 0.25) (layer F.Cu) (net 5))
 (segment (start 128.27 139.38) (end 128.27 137.16) (width 0.25) (layer F.Cu) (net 5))
 (via (at 128.27 137.16) (size 0.6) (drill 0.4) (layers F.Cu B.Cu) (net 5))
 (segment (start 129.54 127.52) (end 129.74 127.52) (width 0.25) (layer F.Cu) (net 5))
 (segment (start 129.74 127.52) (end 137.16 127.52) (width 0.25) (layer F.Cu) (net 5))
 (segment (start 129.54 140.45) (end 137.16 140.45) (width 0.25) (layer F.Cu) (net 5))
 (segment (start 158.75 128.27) (end 152.4 121.92) (width 0.25) (layer F.Cu) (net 6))
 (segment (start 152.4 121.92) (end 144.78 121.92) (width 0.25) (layer F.Cu) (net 6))
 (segment (start 142.24 121.92) (end 143.428601 120.731399) (width 0.25) (layer B.Cu) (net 7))
 (segment (start 143.428601 120.731399) (end 157.956401 120.731399) (width 0.25) (layer B.Cu) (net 7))
 (segment (start 157.956401 120.731399) (end 159.875001 122.649999) (width 0.25) (layer B.Cu) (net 7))
 (segment (start 159.875001 122.649999) (end 159.875001 124.604999) (width 0.25) (layer B.Cu) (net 7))
 (segment (start 159.875001 124.604999) (end 159.549999 124.930001) (width 0.25) (layer B.Cu) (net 7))
 (segment (start 159.549999 124.930001) (end 158.75 125.73) (width 0.25) (layer B.Cu) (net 7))
 (segment (start 142.24 124.46) (end 143.428601 123.271399) (width 0.25) (layer F.Cu) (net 8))
 (segment (start 143.428601 123.271399) (end 149.256399 123.271399) (width 0.25) (layer F.Cu) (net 8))
 (segment (start 149.256399 123.271399) (end 150.589999 124.604999) (width 0.25) (layer F.Cu) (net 8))
 (segment (start 157.950001 130.010001) (end 158.75 130.81) (width 0.25) (layer F.Cu) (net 8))
 (segment (start 150.589999 124.604999) (end 152.544999 124.604999) (width 0.25) (layer F.Cu) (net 8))
 (segment (start 152.544999 124.604999) (end 157.950001 130.010001) (width 0.25) (layer F.Cu) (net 8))
 (segment (start 137.275 121.92) (end 139.7 121.92) (width 0.25) (layer F.Cu) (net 9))
 (segment (start 139.7 121.92) (end 140.97 123.19) (width 0.25) (layer B.Cu) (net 9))
 (segment (start 140.97 123.19) (end 151.13 123.19) (width 0.25) (layer B.Cu) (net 9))
 (segment (start 147.4343 143.51) (end 147.4343 142.86122) (width 0.25) (layer F.Cu) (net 10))
 (segment (start 147.4343 142.86122) (end 149.32552 140.97) (width 0.25) (layer F.Cu) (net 10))
 (segment (start 149.32552 140.97) (end 149.99863 140.97) (width 0.25) (layer F.Cu) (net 10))
 (segment (start 149.99863 140.97) (end 151.13 140.97) (width 0.25) (layer F.Cu) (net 10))
 (segment (start 143.625 143.51) (end 145.9357 143.51) (width 0.25) (layer F.Cu) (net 11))
 (segment (start 147.4343 147.32) (end 147.4343 146.67122) (width 0.25) (layer F.Cu) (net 12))
 (segment (start 147.4343 146.67122) (end 150.59552 143.51) (width 0.25) (layer F.Cu) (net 12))
 (segment (start 150.59552 143.51) (end 151.13 143.51) (width 0.25) (layer F.Cu) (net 12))
 (segment (start 145.9357 147.32) (end 143.625 147.32) (width 0.25) (layer F.Cu) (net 13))
 (segment (start 151.13 125.73) (end 144.145 132.715) (width 0.25) (layer F.Cu) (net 14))
 (segment (start 144.145 132.715) (end 137.32 132.715) (width 0.25) (layer F.Cu) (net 14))
 (segment (start 140.335 133.985) (end 140.335 132.08) (width 0.25) (layer B.Cu) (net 15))
 (segment (start 140.335 132.08) (end 144.145 128.27) (width 0.25) (layer B.Cu) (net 15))
 (segment (start 144.145 128.27) (end 149.99863 128.27) (width 0.25) (layer B.Cu) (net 15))
 (segment (start 149.99863 128.27) (end 151.13 128.27) (width 0.25) (layer B.Cu) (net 15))
 (segment (start 137.32 136.525) (end 136.845 136.525) (width 0.25) (layer F.Cu) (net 15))
 (segment (start 136.845 136.525) (end 136.219999 135.899999) (width 0.25) (layer F.Cu) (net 15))
 (segment (start 136.219999 135.899999) (end 136.219999 134.694999) (width 0.25) (layer F.Cu) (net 15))
 (via (at 140.335 133.985) (size 0.6) (drill 0.4) (layers F.Cu B.Cu) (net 15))
 (segment (start 136.219999 134.694999) (end 136.284999 134.629999) (width 0.25) (layer F.Cu) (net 15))
 (segment (start 136.284999 134.629999) (end 139.690001 134.629999) (width 0.25) (layer F.Cu) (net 15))
 (segment (start 139.690001 134.629999) (end 140.335 133.985) (width 0.25) (layer F.Cu) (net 15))
 (segment (start 130.81 144.78) (end 130.81 146.046) (width 0.25) (layer B.Cu) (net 16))
 (segment (start 130.81 146.046) (end 130.885001 146.121001) (width 0.25) (layer B.Cu) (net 16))
 (segment (start 130.885001 146.121001) (end 140.898999 146.121001) (width 0.25) (layer B.Cu) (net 16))
 (segment (start 140.898999 146.121001) (end 150.330001 136.689999) (width 0.25) (layer B.Cu) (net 16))
 (segment (start 150.330001 136.689999) (end 151.13 135.89) (width 0.25) (layer B.Cu) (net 16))
 (segment (start 145.288 139.7) (end 146.558 138.43) (width 0.25) (layer F.Cu) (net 17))
 (segment (start 146.558 138.43) (end 151.13 138.43) (width 0.25) (layer F.Cu) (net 17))
 (segment (start 141.224 142.24) (end 142.748 142.24) (width 0.25) (layer B.Cu) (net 17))
 (segment (start 142.748 142.24) (end 145.288 139.7) (width 0.25) (layer B.Cu) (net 17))
 (via (at 145.288 139.7) (size 0.6) (drill 0.4) (layers F.Cu B.Cu) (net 17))
 (segment (start 128.27 144.78) (end 128.27 144.6276) (width 0.25) (layer F.Cu) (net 17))
 (segment (start 128.27 144.6276) (end 130.6576 142.24) (width 0.25) (layer F.Cu) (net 17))
 (segment (start 130.6576 142.24) (end 131.516652 142.24) (width 0.25) (layer F.Cu) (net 17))
 (segment (start 131.516652 142.24) (end 141.224 142.24) (width 0.25) (layer F.Cu) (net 17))
 (via (at 141.224 142.24) (size 0.6) (drill 0.4) (layers F.Cu B.Cu) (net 17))
 (segment (start 128.27 144.78) (end 128.27 144.9324) (width 0.25) (layer F.Cu) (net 17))
 (segment (start 130.29 147.955) (end 130.29 147.255) (width 0.25) (layer B.Cu) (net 19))
 (segment (start 130.29 147.255) (end 129.62139 146.58639) (width 0.25) (layer B.Cu) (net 19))
 (segment (start 129.62139 146.58639) (end 129.62139 144.135262) (width 0.25) (layer B.Cu) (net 19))
 (segment (start 129.62139 144.135262) (end 130.317662 143.43899) (width 0.25) (layer B.Cu) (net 19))
 (segment (start 130.317662 143.43899) (end 132.16139 143.43899) (width 0.25) (layer B.Cu) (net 19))
 (segment (start 132.16139 143.43899) (end 133.35 144.6276) (width 0.25) (layer B.Cu) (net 19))
 (segment (start 133.35 144.6276) (end 133.35 144.78) (width 0.25) (layer B.Cu) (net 19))
 (segment (start 158.75 143.51) (end 157.61863 143.51) (width 0.25) (layer F.Cu) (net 19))
 (segment (start 157.61863 143.51) (end 153.033629 148.095001) (width 0.25) (layer F.Cu) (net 19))
 (segment (start 153.033629 148.095001) (end 136.512601 148.095001) (width 0.25) (layer F.Cu) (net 19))
 (segment (start 133.35 144.9324) (end 133.35 144.78) (width 0.25) (layer F.Cu) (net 19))
 (segment (start 136.512601 148.095001) (end 133.35 144.9324) (width 0.25) (layer F.Cu) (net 19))
 (segment (start 133.35 144.78) (end 133.35 144.6276) (width 0.25) (layer F.Cu) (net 19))
 (segment (start 158.75 140.97) (end 157.624999 139.844999) (width 0.25) (layer F.Cu) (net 20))
 (segment (start 151.380003 129.395001) (end 149.080001 129.395001) (width 0.25) (layer F.Cu) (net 20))
 (segment (start 157.624999 139.844999) (end 157.624999 135.639997) (width 0.25) (layer F.Cu) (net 20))
 (segment (start 157.624999 135.639997) (end 151.380003 129.395001) (width 0.25) (layer F.Cu) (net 20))
 (segment (start 140.888601 126.576401) (end 140.888601 123.889471) (width 0.25) (layer F.Cu) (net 20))
 (segment (start 140.168809 123.169679) (end 132.694679 123.169679) (width 0.25) (layer F.Cu) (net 20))
 (segment (start 149.080001 129.395001) (end 145.135001 133.340001) (width 0.25) (layer F.Cu) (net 20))
 (segment (start 145.135001 133.340001) (end 136.284999 133.340001) (width 0.25) (layer F.Cu) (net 20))
 (segment (start 136.219999 133.275001) (end 136.219999 131.245003) (width 0.25) (layer F.Cu) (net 20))
 (segment (start 136.219999 131.245003) (end 140.888601 126.576401) (width 0.25) (layer F.Cu) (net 20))
 (segment (start 136.284999 133.340001) (end 136.219999 133.275001) (width 0.25) (layer F.Cu) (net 20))
 (segment (start 140.888601 123.889471) (end 140.168809 123.169679) (width 0.25) (layer F.Cu) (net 20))
 (segment (start 132.694679 123.169679) (end 131.445 121.92) (width 0.25) (layer F.Cu) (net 20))
 (segment (start 125.476 128.766) (end 125.476 130.556) (width 0.25) (layer B.Cu) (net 24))
 (segment (start 125.476 130.556) (end 125.73 130.81) (width 0.25) (layer B.Cu) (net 24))
 (segment (start 123.19 132.08) (end 124.46 130.81) (width 0.25) (layer F.Cu) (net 24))
 (segment (start 124.46 130.81) (end 125.73 130.81) (width 0.25) (layer F.Cu) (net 24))
 (segment (start 129.54 132.08) (end 127 132.08) (width 0.25) (layer F.Cu) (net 25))
 (segment (start 127 132.08) (end 125.73 133.35) (width 0.25) (layer F.Cu) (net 25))
 (segment (start 129.54 129.02) (end 137.16 129.02) (width 0.25) (layer F.Cu) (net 25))
 (segment (start 131.92 133.985) (end 131.445 133.985) (width 0.25) (layer F.Cu) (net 25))
 (segment (start 131.445 133.985) (end 129.54 132.08) (width 0.25) (layer F.Cu) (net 25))
 (segment (start 129.54 132.08) (end 129.54 129.52) (width 0.25) (layer F.Cu) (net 25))
 (segment (start 129.54 129.52) (end 129.54 129.02) (width 0.25) (layer F.Cu) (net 25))
 (segment (start 127 134.62) (end 129.54 137.16) (width 0.25) (layer F.Cu) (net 26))
 (segment (start 123.19 134.62) (end 127 134.62) (width 0.25) (layer F.Cu) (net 26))
 (segment (start 129.54 138.95) (end 137.16 138.95) (width 0.25) (layer F.Cu) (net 26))
 (segment (start 129.54 138.95) (end 129.54 137.16) (width 0.25) (layer F.Cu) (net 26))
 (segment (start 129.54 137.16) (end 131.445 135.255) (width 0.25) (layer F.Cu) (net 26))
 (segment (start 131.445 135.255) (end 131.92 135.255) (width 0.25) (layer F.Cu) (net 26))
 (segment (start 123.19 137.16) (end 123.19 140.696) (width 0.25) (layer B.Cu) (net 27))
 (segment (start 123.19 140.696) (end 123.21 140.716) (width 0.25) (layer B.Cu) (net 27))
 (segment (start 123.21 140.716) (end 123.71 140.716) (width 0.25) (layer B.Cu) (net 27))
 (segment (start 123.19 142.22) (end 123.21 142.24) (width 0.25) (layer B.Cu) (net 27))
 (segment (start 123.19 137.16) (end 124.46 135.89) (width 0.25) (layer F.Cu) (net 27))
 (segment (start 124.46 135.89) (end 125.73 135.89) (width 0.25) (layer F.Cu) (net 27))
 (segment (start 133.87 125.73) (end 132.715 125.73) (width 0.25) (layer B.Cu) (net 28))
 (segment (start 132.715 125.73) (end 126.40564 119.42064) (width 0.25) (layer B.Cu) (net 28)))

